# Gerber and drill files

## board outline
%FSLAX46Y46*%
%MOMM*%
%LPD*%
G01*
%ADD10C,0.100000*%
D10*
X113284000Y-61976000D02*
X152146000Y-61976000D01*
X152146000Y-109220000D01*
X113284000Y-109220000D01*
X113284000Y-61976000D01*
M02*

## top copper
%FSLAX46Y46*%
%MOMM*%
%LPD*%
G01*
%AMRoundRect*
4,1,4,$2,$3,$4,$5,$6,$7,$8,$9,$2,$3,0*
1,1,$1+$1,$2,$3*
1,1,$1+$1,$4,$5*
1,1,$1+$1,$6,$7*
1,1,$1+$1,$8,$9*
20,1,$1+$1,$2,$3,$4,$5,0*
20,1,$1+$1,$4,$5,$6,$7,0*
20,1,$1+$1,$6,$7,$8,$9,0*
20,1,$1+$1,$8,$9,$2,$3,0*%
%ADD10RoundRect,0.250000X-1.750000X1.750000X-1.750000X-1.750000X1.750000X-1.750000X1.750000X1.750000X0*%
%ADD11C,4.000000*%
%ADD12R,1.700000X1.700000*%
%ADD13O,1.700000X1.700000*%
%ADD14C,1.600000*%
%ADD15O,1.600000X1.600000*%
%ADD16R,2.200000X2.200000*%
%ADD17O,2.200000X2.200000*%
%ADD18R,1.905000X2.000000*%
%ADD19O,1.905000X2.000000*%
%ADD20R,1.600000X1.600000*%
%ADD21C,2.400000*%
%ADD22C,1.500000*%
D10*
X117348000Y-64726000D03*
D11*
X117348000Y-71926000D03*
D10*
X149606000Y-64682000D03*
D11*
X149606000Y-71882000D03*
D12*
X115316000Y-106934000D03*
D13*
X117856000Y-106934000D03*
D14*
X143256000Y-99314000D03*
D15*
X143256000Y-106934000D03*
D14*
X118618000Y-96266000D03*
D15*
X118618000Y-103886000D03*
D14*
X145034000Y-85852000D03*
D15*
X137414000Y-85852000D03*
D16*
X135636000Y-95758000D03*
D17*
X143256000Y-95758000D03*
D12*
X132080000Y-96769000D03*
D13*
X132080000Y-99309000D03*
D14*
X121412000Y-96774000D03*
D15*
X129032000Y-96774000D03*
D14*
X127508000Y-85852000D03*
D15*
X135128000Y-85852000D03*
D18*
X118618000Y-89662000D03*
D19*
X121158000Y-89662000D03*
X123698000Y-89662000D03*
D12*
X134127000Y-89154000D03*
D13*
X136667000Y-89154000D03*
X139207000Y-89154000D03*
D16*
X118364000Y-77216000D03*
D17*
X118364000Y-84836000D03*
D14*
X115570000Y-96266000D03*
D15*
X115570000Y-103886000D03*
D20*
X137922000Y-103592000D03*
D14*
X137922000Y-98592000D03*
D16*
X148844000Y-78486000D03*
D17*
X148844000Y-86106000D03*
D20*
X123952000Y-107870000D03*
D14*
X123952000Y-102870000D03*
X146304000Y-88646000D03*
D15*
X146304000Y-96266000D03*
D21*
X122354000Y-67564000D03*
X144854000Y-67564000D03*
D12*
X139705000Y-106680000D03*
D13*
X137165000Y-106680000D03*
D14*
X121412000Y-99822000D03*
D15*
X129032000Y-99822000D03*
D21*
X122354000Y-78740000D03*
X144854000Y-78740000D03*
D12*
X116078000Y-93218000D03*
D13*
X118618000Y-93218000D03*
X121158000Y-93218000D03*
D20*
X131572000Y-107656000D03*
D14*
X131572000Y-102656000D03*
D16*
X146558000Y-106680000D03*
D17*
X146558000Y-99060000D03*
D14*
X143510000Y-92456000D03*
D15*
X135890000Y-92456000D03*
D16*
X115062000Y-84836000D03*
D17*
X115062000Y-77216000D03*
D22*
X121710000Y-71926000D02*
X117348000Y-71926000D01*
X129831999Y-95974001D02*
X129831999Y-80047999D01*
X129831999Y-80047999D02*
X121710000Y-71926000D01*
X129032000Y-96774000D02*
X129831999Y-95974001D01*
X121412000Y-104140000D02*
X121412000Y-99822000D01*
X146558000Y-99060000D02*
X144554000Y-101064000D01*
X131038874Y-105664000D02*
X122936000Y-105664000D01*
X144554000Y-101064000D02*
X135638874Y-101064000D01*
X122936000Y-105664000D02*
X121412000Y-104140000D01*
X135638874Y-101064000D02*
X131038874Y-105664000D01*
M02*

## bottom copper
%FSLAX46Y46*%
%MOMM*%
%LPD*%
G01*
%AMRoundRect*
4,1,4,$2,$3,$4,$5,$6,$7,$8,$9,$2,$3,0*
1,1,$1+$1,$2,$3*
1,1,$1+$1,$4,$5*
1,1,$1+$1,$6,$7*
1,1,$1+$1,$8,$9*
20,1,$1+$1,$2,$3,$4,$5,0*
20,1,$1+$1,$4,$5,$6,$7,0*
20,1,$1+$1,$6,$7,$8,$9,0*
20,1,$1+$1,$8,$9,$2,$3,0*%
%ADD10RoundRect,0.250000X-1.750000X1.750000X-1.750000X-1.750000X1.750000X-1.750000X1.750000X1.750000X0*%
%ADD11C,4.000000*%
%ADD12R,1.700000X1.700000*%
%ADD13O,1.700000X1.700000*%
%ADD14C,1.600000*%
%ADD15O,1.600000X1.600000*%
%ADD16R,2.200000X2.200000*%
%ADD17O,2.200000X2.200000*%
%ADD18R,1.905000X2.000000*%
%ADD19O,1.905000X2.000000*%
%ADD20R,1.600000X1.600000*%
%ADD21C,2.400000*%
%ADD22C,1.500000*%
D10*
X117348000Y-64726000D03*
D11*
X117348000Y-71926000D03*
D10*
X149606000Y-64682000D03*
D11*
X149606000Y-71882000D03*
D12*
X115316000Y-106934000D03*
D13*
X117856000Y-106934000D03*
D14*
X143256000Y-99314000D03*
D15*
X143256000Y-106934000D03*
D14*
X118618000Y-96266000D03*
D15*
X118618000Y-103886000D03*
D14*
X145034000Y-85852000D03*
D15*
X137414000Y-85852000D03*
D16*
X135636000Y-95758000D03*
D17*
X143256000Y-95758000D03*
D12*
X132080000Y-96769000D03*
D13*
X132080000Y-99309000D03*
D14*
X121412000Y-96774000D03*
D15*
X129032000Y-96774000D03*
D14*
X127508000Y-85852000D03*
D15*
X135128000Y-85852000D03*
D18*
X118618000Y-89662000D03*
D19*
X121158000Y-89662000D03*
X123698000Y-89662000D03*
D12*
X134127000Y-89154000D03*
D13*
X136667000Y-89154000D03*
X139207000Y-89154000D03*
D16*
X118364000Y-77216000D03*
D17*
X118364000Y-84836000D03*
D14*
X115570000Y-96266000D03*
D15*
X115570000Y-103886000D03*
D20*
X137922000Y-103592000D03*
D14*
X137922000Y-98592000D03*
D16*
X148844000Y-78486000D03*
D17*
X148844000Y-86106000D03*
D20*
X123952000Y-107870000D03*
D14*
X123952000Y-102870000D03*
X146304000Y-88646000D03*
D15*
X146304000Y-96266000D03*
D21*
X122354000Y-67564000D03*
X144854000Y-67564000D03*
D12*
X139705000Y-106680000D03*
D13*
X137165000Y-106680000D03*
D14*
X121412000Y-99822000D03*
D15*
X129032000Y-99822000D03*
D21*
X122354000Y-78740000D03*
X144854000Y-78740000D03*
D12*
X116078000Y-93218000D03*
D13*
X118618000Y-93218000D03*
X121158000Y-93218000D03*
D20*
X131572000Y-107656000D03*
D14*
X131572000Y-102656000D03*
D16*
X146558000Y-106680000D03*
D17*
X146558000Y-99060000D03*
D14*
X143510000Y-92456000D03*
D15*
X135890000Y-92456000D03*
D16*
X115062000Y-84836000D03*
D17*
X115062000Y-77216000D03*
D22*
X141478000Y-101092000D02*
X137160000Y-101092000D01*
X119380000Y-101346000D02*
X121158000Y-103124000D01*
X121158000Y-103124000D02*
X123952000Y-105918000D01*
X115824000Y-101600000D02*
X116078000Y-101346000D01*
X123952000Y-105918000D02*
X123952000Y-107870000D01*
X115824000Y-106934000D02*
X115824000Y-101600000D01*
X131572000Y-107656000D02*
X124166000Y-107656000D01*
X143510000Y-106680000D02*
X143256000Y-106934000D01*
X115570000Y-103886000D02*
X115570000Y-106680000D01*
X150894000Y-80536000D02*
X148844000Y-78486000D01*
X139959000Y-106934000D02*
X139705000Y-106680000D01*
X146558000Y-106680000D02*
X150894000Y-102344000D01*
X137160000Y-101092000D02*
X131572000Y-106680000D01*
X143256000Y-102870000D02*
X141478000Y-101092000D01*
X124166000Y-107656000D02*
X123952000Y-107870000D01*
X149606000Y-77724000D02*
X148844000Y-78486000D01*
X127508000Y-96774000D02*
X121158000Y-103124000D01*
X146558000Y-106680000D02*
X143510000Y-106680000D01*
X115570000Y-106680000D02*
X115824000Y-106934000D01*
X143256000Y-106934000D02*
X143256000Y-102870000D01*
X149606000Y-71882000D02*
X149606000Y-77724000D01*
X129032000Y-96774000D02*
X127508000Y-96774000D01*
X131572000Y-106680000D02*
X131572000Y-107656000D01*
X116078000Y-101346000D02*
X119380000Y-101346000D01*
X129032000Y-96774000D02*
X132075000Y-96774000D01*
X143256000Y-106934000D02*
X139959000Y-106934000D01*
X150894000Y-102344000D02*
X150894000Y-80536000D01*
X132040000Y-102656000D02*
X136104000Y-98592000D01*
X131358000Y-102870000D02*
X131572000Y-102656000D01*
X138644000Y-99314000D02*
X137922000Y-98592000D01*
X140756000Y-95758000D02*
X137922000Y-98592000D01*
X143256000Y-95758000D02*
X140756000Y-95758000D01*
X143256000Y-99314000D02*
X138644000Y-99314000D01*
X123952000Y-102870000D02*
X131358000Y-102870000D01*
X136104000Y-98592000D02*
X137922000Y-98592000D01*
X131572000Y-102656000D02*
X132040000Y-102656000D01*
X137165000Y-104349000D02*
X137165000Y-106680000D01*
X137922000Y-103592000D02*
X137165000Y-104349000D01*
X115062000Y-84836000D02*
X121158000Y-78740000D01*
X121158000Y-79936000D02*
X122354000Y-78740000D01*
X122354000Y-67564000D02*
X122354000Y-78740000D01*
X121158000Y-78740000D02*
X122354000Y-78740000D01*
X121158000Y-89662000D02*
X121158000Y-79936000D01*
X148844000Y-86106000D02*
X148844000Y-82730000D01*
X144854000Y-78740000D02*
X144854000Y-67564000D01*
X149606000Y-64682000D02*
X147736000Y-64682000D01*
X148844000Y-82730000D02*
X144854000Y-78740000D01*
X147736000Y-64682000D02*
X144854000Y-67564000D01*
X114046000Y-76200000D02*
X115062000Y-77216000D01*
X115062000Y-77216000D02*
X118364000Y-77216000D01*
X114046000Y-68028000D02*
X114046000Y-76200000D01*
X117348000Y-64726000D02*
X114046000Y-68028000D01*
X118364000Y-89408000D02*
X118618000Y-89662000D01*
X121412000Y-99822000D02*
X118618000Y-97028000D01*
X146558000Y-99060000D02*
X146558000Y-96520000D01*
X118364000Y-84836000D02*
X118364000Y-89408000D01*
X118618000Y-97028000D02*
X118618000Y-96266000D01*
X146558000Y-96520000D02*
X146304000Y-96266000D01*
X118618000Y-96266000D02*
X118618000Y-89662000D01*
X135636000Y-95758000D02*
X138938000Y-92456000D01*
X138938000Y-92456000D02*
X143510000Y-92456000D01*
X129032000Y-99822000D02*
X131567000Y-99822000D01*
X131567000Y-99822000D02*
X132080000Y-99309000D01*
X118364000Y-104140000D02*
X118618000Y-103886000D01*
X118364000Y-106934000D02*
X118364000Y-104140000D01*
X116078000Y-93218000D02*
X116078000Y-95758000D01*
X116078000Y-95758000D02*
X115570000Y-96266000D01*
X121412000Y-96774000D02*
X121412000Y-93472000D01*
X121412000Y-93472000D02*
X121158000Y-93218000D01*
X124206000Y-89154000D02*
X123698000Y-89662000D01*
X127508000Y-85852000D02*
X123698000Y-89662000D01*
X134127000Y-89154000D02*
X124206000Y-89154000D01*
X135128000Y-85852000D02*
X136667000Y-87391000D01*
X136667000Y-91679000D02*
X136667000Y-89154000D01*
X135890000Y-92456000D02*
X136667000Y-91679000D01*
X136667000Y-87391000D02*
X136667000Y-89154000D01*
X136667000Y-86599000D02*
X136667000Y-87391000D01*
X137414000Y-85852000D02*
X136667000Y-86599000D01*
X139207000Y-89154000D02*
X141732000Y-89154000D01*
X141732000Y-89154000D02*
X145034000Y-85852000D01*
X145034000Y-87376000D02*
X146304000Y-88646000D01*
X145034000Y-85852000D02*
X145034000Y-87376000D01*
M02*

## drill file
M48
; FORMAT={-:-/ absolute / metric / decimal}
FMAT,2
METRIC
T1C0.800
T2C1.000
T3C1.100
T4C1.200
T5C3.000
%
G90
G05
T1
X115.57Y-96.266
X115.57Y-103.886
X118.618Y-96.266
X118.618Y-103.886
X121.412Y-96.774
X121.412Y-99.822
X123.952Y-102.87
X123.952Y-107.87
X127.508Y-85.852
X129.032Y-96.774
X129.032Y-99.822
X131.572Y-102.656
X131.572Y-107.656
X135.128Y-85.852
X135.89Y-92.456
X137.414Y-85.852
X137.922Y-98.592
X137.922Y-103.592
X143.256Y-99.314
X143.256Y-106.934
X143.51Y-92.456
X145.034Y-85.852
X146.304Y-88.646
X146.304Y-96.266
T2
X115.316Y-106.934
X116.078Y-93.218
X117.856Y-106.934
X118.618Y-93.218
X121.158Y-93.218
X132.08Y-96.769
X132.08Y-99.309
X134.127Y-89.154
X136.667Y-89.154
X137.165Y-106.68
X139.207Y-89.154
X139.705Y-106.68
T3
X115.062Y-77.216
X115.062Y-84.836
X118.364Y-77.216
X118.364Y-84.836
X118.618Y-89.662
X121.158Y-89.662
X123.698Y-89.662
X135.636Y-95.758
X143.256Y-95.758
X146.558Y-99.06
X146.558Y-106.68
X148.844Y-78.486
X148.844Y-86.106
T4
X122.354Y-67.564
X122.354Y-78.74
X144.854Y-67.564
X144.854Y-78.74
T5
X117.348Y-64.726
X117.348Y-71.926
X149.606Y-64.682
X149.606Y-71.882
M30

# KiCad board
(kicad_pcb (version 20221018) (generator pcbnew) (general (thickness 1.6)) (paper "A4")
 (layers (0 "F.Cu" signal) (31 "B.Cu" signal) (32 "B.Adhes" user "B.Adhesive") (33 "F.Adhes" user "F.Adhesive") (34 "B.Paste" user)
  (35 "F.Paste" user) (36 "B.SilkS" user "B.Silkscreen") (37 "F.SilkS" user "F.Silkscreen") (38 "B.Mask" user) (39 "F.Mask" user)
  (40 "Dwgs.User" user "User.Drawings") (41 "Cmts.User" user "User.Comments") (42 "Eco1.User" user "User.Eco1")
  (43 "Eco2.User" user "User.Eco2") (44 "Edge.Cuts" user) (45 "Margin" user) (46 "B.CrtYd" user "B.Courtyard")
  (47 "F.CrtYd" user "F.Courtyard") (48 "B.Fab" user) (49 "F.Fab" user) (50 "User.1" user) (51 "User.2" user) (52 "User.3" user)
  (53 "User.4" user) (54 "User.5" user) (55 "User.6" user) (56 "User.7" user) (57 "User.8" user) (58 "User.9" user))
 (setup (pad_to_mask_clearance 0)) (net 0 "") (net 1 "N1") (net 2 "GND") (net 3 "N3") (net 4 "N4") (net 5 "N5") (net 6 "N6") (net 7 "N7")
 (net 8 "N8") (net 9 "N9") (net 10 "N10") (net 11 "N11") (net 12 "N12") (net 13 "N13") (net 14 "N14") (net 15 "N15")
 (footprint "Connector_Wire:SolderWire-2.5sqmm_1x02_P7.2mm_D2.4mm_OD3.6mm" (layer "F.Cu") (at 117.348 64.726 -90)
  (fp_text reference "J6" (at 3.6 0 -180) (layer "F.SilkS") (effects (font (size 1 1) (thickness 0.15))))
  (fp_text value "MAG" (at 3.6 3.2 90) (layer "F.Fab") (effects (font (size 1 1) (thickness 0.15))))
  (pad "1" thru_hole roundrect (at 0 0 270) (size 4 4) (drill 3) (layers "*.Cu" "*.Mask") (roundrect_rratio 0.0625) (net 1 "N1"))
  (pad "2" thru_hole circle (at 7.2 0 270) (size 4 4) (drill 3) (layers "*.Cu" "*.Mask") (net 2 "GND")))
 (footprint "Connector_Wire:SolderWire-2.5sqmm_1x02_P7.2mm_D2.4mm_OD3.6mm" (layer "F.Cu") (at 149.606 64.682 -90)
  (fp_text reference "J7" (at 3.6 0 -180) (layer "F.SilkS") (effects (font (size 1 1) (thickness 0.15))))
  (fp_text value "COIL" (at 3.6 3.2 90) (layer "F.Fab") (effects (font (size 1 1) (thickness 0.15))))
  (pad "1" thru_hole roundrect (at 0 0 270) (size 4 4) (drill 3) (layers "*.Cu" "*.Mask") (roundrect_rratio 0.0625) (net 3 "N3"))
  (pad "2" thru_hole circle (at 7.2 0 270) (size 4 4) (drill 3) (layers "*.Cu" "*.Mask") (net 2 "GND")))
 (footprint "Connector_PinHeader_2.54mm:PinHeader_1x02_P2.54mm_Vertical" (layer "F.Cu") (at 115.316 106.934 90)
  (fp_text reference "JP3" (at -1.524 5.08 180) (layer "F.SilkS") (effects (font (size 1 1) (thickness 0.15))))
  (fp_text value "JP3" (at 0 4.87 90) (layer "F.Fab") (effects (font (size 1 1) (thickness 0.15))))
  (pad "1" thru_hole rect (at 0 0 90) (size 1.7 1.7) (drill 1) (layers "*.Cu" "*.Mask") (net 2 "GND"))
  (pad "2" thru_hole oval (at 0 2.54 90) (size 1.7 1.7) (drill 1) (layers "*.Cu" "*.Mask") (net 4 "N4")))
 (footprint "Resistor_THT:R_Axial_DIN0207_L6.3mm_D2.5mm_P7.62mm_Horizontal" (layer "F.Cu") (at 143.256 99.314 -90)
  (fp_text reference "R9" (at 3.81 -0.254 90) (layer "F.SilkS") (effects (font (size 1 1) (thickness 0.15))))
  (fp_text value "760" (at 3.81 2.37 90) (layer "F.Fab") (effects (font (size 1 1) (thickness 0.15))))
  (pad "1" thru_hole circle (at 0 0 270) (size 1.6 1.6) (drill 0.8) (layers "*.Cu" "*.Mask") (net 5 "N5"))
  (pad "2" thru_hole oval (at 7.62 0 270) (size 1.6 1.6) (drill 0.8) (layers "*.Cu" "*.Mask") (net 2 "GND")))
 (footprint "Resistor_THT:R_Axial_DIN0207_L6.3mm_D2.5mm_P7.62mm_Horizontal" (layer "F.Cu") (at 118.618 96.266 -90)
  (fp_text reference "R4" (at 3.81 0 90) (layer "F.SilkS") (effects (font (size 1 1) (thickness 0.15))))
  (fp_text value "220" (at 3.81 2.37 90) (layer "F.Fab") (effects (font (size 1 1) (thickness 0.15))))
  (pad "1" thru_hole circle (at 0 0 270) (size 1.6 1.6) (drill 0.8) (layers "*.Cu" "*.Mask") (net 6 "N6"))
  (pad "2" thru_hole oval (at 7.62 0 270) (size 1.6 1.6) (drill 0.8) (layers "*.Cu" "*.Mask") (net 4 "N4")))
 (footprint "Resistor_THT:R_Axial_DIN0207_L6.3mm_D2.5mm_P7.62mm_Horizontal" (layer "F.Cu") (at 145.034 85.852 180)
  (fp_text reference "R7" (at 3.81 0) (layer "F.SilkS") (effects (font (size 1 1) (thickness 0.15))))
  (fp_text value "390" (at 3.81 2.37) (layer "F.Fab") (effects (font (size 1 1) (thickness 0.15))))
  (pad "1" thru_hole circle (at 0 0 180) (size 1.6 1.6) (drill 0.8) (layers "*.Cu" "*.Mask") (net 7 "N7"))
  (pad "2" thru_hole oval (at 7.62 0 180) (size 1.6 1.6) (drill 0.8) (layers "*.Cu" "*.Mask") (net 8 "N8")))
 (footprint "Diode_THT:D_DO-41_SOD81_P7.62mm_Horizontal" (layer "F.Cu") (at 135.636 95.758)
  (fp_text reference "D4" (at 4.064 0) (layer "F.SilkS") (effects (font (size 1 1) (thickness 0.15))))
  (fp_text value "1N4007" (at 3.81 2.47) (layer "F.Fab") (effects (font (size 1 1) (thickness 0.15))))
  (pad "1" thru_hole rect (at 0 0) (size 2.2 2.2) (drill 1.1) (layers "*.Cu" "*.Mask") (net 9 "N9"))
  (pad "2" thru_hole oval (at 7.62 0) (size 2.2 2.2) (drill 1.1) (layers "*.Cu" "*.Mask") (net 5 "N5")))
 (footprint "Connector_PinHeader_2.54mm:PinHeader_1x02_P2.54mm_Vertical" (layer "F.Cu") (at 132.08 96.769)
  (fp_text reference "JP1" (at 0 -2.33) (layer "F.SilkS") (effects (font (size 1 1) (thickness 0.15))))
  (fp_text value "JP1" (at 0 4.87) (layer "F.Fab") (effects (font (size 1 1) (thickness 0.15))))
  (pad "1" thru_hole rect (at 0 0) (size 1.7 1.7) (drill 1) (layers "*.Cu" "*.Mask") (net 2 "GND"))
  (pad "2" thru_hole oval (at 0 2.54) (size 1.7 1.7) (drill 1) (layers "*.Cu" "*.Mask") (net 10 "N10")))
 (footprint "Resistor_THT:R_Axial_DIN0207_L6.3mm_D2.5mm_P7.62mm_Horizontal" (layer "F.Cu") (at 121.412 96.774)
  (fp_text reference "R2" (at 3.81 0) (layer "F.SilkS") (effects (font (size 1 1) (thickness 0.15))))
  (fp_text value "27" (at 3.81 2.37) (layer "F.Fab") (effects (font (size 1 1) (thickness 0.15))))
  (pad "1" thru_hole circle (at 0 0) (size 1.6 1.6) (drill 0.8) (layers "*.Cu" "*.Mask") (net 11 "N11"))
  (pad "2" thru_hole oval (at 7.62 0) (size 1.6 1.6) (drill 0.8) (layers "*.Cu" "*.Mask") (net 2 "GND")))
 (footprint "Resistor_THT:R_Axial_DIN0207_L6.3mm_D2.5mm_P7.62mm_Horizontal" (layer "F.Cu") (at 127.508 85.852)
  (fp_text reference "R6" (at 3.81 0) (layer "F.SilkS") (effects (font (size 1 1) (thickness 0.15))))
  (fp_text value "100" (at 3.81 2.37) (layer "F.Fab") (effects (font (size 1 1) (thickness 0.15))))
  (pad "1" thru_hole circle (at 0 0) (size 1.6 1.6) (drill 0.8) (layers "*.Cu" "*.Mask") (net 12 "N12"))
  (pad "2" thru_hole oval (at 7.62 0) (size 1.6 1.6) (drill 0.8) (layers "*.Cu" "*.Mask") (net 8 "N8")))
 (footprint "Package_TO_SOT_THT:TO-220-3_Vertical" (layer "F.Cu") (at 118.618 89.662)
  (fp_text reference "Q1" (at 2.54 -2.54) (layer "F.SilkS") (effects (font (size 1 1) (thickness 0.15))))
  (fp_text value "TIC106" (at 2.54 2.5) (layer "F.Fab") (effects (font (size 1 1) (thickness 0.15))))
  (pad "1" thru_hole rect (at 0 0) (size 1.905 2) (drill 1.1) (layers "*.Cu" "*.Mask") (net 6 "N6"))
  (pad "2" thru_hole oval (at 2.54 0) (size 1.905 2) (drill 1.1) (layers "*.Cu" "*.Mask") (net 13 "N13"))
  (pad "3" thru_hole oval (at 5.08 0) (size 1.905 2) (drill 1.1) (layers "*.Cu" "*.Mask") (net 12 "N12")))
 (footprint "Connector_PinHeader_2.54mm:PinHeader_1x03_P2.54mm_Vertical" (layer "F.Cu") (at 134.127 89.154 90)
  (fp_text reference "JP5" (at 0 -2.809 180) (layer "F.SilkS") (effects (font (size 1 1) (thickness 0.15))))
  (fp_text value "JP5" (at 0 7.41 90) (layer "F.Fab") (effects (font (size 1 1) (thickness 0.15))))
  (pad "1" thru_hole rect (at 0 0 90) (size 1.7 1.7) (drill 1) (layers "*.Cu" "*.Mask") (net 12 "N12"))
  (pad "2" thru_hole oval (at 0 2.54 90) (size 1.7 1.7) (drill 1) (layers "*.Cu" "*.Mask") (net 8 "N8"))
  (pad "3" thru_hole oval (at 0 5.08 90) (size 1.7 1.7) (drill 1) (layers "*.Cu" "*.Mask") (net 7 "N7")))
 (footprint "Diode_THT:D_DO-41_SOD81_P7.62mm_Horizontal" (layer "F.Cu") (at 118.364 77.216 -90)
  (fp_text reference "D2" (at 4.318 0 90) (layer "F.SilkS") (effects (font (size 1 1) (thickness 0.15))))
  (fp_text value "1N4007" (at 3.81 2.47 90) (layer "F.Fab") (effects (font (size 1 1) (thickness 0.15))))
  (pad "1" thru_hole rect (at 0 0 270) (size 2.2 2.2) (drill 1.1) (layers "*.Cu" "*.Mask") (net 1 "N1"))
  (pad "2" thru_hole oval (at 7.62 0 270) (size 2.2 2.2) (drill 1.1) (layers "*.Cu" "*.Mask") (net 6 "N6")))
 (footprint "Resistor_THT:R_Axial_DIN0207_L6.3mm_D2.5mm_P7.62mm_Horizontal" (layer "F.Cu") (at 115.57 96.266 -90)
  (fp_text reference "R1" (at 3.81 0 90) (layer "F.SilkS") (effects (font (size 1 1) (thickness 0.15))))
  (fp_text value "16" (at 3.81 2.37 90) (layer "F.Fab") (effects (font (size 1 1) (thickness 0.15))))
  (pad "1" thru_hole circle (at 0 0 270) (size 1.6 1.6) (drill 0.8) (layers "*.Cu" "*.Mask") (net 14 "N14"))
  (pad "2" thru_hole oval (at 7.62 0 270) (size 1.6 1.6) (drill 0.8) (layers "*.Cu" "*.Mask") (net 2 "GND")))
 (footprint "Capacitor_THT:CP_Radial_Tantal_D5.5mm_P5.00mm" (layer "F.Cu") (at 137.922 103.592 90)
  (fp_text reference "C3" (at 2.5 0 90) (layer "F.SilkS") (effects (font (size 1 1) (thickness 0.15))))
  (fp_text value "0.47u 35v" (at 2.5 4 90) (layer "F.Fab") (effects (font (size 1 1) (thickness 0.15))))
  (pad "1" thru_hole rect (at 0 0 90) (size 1.6 1.6) (drill 0.8) (layers "*.Cu" "*.Mask") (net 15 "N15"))
  (pad "2" thru_hole circle (at 5 0 90) (size 1.6 1.6) (drill 0.8) (layers "*.Cu" "*.Mask") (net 5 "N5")))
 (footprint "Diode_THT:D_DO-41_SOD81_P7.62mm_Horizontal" (layer "F.Cu") (at 148.844 78.486 -90)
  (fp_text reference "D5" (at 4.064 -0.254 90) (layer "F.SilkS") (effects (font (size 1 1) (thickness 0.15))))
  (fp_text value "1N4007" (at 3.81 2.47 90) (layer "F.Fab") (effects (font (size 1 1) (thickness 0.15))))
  (pad "1" thru_hole rect (at 0 0 270) (size 2.2 2.2) (drill 1.1) (layers "*.Cu" "*.Mask") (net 2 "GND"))
  (pad "2" thru_hole oval (at 7.62 0 270) (size 2.2 2.2) (drill 1.1) (layers "*.Cu" "*.Mask") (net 3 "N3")))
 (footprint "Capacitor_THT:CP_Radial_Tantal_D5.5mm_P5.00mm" (layer "F.Cu") (at 123.952 107.87 90)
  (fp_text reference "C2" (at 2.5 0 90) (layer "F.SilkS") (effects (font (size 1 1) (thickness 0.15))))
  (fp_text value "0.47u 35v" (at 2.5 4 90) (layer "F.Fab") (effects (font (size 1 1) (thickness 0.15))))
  (pad "1" thru_hole rect (at 0 0 90) (size 1.6 1.6) (drill 0.8) (layers "*.Cu" "*.Mask") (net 2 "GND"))
  (pad "2" thru_hole circle (at 5 0 90) (size 1.6 1.6) (drill 0.8) (layers "*.Cu" "*.Mask") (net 5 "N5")))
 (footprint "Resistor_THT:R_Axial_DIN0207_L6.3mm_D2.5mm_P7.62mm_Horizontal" (layer "F.Cu") (at 146.304 88.646 -90)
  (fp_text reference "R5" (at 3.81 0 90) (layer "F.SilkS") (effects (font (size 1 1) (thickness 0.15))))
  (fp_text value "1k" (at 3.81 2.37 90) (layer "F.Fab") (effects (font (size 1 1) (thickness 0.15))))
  (pad "1" thru_hole circle (at 0 0 270) (size 1.6 1.6) (drill 0.8) (layers "*.Cu" "*.Mask") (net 7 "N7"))
  (pad "2" thru_hole oval (at 7.62 0 270) (size 1.6 1.6) (drill 0.8) (layers "*.Cu" "*.Mask") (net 6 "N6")))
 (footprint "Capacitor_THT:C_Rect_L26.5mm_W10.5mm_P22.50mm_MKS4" (layer "F.Cu") (at 122.354 67.564)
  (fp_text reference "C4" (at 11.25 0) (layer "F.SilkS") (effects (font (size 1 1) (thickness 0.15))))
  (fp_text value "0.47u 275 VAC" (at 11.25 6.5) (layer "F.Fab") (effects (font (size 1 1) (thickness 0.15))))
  (pad "1" thru_hole circle (at 0 0) (size 2.4 2.4) (drill 1.2) (layers "*.Cu" "*.Mask") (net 13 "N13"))
  (pad "2" thru_hole circle (at 22.5 0) (size 2.4 2.4) (drill 1.2) (layers "*.Cu" "*.Mask") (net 3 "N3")))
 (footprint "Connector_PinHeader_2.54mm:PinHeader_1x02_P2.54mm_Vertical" (layer "F.Cu") (at 139.705 106.68 -90)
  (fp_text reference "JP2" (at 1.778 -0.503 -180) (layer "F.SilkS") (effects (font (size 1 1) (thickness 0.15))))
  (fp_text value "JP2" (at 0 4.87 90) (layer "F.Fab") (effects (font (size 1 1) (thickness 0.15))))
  (pad "1" thru_hole rect (at 0 0 270) (size 1.7 1.7) (drill 1) (layers "*.Cu" "*.Mask") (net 2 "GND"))
  (pad "2" thru_hole oval (at 0 2.54 270) (size 1.7 1.7) (drill 1) (layers "*.Cu" "*.Mask") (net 15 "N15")))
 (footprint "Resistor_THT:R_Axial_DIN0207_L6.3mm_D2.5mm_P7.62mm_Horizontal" (layer "F.Cu") (at 121.412 99.822)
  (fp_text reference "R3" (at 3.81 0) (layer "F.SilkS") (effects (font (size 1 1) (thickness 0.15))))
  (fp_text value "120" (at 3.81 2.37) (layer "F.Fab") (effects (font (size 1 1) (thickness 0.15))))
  (pad "1" thru_hole circle (at 0 0) (size 1.6 1.6) (drill 0.8) (layers "*.Cu" "*.Mask") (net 6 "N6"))
  (pad "2" thru_hole oval (at 7.62 0) (size 1.6 1.6) (drill 0.8) (layers "*.Cu" "*.Mask") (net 10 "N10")))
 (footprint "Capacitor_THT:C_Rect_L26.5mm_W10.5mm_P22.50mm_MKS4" (layer "F.Cu") (at 122.354 78.74)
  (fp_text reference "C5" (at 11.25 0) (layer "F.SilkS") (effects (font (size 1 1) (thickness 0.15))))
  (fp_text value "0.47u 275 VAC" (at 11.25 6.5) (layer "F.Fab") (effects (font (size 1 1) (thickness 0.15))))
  (pad "1" thru_hole circle (at 0 0) (size 2.4 2.4) (drill 1.2) (layers "*.Cu" "*.Mask") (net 13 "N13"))
  (pad "2" thru_hole circle (at 22.5 0) (size 2.4 2.4) (drill 1.2) (layers "*.Cu" "*.Mask") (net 3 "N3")))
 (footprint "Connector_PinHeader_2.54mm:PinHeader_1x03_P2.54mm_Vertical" (layer "F.Cu") (at 116.078 93.218 90)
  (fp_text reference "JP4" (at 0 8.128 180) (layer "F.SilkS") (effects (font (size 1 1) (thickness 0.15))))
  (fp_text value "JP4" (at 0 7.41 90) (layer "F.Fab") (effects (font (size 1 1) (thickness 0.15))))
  (pad "1" thru_hole rect (at 0 0 90) (size 1.7 1.7) (drill 1) (layers "*.Cu" "*.Mask") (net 14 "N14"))
  (pad "2" thru_hole oval (at 0 2.54 90) (size 1.7 1.7) (drill 1) (layers "*.Cu" "*.Mask") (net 6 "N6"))
  (pad "3" thru_hole oval (at 0 5.08 90) (size 1.7 1.7) (drill 1) (layers "*.Cu" "*.Mask") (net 11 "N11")))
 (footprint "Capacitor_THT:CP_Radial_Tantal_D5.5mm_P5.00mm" (layer "F.Cu") (at 131.572 107.656 90)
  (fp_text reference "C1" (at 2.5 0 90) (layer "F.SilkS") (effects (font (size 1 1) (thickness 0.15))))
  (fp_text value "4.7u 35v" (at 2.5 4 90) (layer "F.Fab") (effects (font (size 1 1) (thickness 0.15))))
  (pad "1" thru_hole rect (at 0 0 90) (size 1.6 1.6) (drill 0.8) (layers "*.Cu" "*.Mask") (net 2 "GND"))
  (pad "2" thru_hole circle (at 5 0 90) (size 1.6 1.6) (drill 0.8) (layers "*.Cu" "*.Mask") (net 5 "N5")))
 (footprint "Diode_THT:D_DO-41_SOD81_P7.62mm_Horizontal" (layer "F.Cu") (at 146.558 106.68 90)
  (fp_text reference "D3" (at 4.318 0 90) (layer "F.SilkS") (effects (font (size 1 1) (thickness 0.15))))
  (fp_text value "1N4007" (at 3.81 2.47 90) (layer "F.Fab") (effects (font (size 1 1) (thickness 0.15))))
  (pad "1" thru_hole rect (at 0 0 90) (size 2.2 2.2) (drill 1.1) (layers "*.Cu" "*.Mask") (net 2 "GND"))
  (pad "2" thru_hole oval (at 7.62 0 90) (size 2.2 2.2) (drill 1.1) (layers "*.Cu" "*.Mask") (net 6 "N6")))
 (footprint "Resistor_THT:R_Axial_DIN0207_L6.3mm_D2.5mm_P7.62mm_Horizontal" (layer "F.Cu") (at 143.51 92.456 180)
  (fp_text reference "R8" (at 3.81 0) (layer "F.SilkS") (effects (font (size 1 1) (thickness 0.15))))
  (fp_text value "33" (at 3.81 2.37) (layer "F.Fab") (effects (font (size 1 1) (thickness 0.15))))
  (pad "1" thru_hole circle (at 0 0 180) (size 1.6 1.6) (drill 0.8) (layers "*.Cu" "*.Mask") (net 9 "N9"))
  (pad "2" thru_hole oval (at 7.62 0 180) (size 1.6 1.6) (drill 0.8) (layers "*.Cu" "*.Mask") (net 8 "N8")))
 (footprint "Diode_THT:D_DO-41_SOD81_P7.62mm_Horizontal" (layer "F.Cu") (at 115.062 84.836 90)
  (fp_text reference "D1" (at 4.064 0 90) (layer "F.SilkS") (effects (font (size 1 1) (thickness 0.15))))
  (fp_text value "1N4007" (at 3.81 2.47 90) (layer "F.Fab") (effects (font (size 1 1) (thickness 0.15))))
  (pad "1" thru_hole rect (at 0 0 90) (size 2.2 2.2) (drill 1.1) (layers "*.Cu" "*.Mask") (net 13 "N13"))
  (pad "2" thru_hole oval (at 7.62 0 90) (size 2.2 2.2) (drill 1.1) (layers "*.Cu" "*.Mask") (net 1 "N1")))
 (gr_rect (start 113.284 61.976) (end 152.146 109.22) (stroke (width 0.1) (type default)) (fill none) (layer "Edge.Cuts"))
 (segment (start 121.71 71.926) (end 117.348 71.926) (width 1.5) (layer "F.Cu") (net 2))
 (segment (start 129.831999 95.974001) (end 129.831999 80.047999) (width 1.5) (layer "F.Cu") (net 2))
 (segment (start 129.831999 80.047999) (end 121.71 71.926) (width 1.5) (layer "F.Cu") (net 2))
 (segment (start 129.032 96.774) (end 129.831999 95.974001) (width 1.5) (layer "F.Cu") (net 2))
 (segment (start 141.478 101.092) (end 137.16 101.092) (width 1.5) (layer "B.Cu") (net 2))
 (segment (start 119.38 101.346) (end 121.158 103.124) (width 1.5) (layer "B.Cu") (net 2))
 (segment (start 121.158 103.124) (end 123.952 105.918) (width 1.5) (layer "B.Cu") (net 2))
 (segment (start 115.824 101.6) (end 116.078 101.346) (width 1.5) (layer "B.Cu") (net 2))
 (segment (start 123.952 105.918) (end 123.952 107.87) (width 1.5) (layer "B.Cu") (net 2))
 (segment (start 115.824 106.934) (end 115.824 101.6) (width 1.5) (layer "B.Cu") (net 2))
 (segment (start 131.572 107.656) (end 124.166 107.656) (width 1.5) (layer "B.Cu") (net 2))
 (segment (start 143.51 106.68) (end 143.256 106.934) (width 1.5) (layer "B.Cu") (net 2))
 (segment (start 115.57 103.886) (end 115.57 106.68) (width 1.5) (layer "B.Cu") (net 2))
 (segment (start 150.894 80.536) (end 148.844 78.486) (width 1.5) (layer "B.Cu") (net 2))
 (segment (start 139.959 106.934) (end 139.705 106.68) (width 1.5) (layer "B.Cu") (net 2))
 (segment (start 146.558 106.68) (end 150.894 102.344) (width 1.5) (layer "B.Cu") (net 2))
 (segment (start 137.16 101.092) (end 131.572 106.68) (width 1.5) (layer "B.Cu") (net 2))
 (segment (start 143.256 102.87) (end 141.478 101.092) (width 1.5) (layer "B.Cu") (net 2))
 (segment (start 124.166 107.656) (end 123.952 107.87) (width 1.5) (layer "B.Cu") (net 2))
 (segment (start 149.606 77.724) (end 148.844 78.486) (width 1.5) (layer "B.Cu") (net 2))
 (segment (start 127.508 96.774) (end 121.158 103.124) (width 1.5) (layer "B.Cu") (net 2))
 (segment (start 146.558 106.68) (end 143.51 106.68) (width 1.5) (layer "B.Cu") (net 2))
 (segment (start 115.57 106.68) (end 115.824 106.934) (width 1.5) (layer "B.Cu") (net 2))
 (segment (start 143.256 106.934) (end 143.256 102.87) (width 1.5) (layer "B.Cu") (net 2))
 (segment (start 149.606 71.882) (end 149.606 77.724) (width 1.5) (layer "B.Cu") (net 2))
 (segment (start 129.032 96.774) (end 127.508 96.774) (width 1.5) (layer "B.Cu") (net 2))
 (segment (start 131.572 106.68) (end 131.572 107.656) (width 1.5) (layer "B.Cu") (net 2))
 (segment (start 116.078 101.346) (end 119.38 101.346) (width 1.5) (layer "B.Cu") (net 2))
 (segment (start 129.032 96.774) (end 132.075 96.774) (width 1.5) (layer "B.Cu") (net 2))
 (segment (start 143.256 106.934) (end 139.959 106.934) (width 1.5) (layer "B.Cu") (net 2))
 (segment (start 150.894 102.344) (end 150.894 80.536) (width 1.5) (layer "B.Cu") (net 2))
 (segment (start 132.04 102.656) (end 136.104 98.592) (width 1.5) (layer "B.Cu") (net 5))
 (segment (start 131.358 102.87) (end 131.572 102.656) (width 1.5) (layer "B.Cu") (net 5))
 (segment (start 138.644 99.314) (end 137.922 98.592) (width 1.5) (layer "B.Cu") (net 5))
 (segment (start 140.756 95.758) (end 137.922 98.592) (width 1.5) (layer "B.Cu") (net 5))
 (segment (start 143.256 95.758) (end 140.756 95.758) (width 1.5) (layer "B.Cu") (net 5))
 (segment (start 143.256 99.314) (end 138.644 99.314) (width 1.5) (layer "B.Cu") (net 5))
 (segment (start 123.952 102.87) (end 131.358 102.87) (width 1.5) (layer "B.Cu") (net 5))
 (segment (start 136.104 98.592) (end 137.922 98.592) (width 1.5) (layer "B.Cu") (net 5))
 (segment (start 131.572 102.656) (end 132.04 102.656) (width 1.5) (layer "B.Cu") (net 5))
 (segment (start 137.165 104.349) (end 137.165 106.68) (width 1.5) (layer "B.Cu") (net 15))
 (segment (start 137.922 103.592) (end 137.165 104.349) (width 1.5) (layer "B.Cu") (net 15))
 (segment (start 115.062 84.836) (end 121.158 78.74) (width 1.5) (layer "B.Cu") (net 13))
 (segment (start 121.158 79.936) (end 122.354 78.74) (width 1.5) (layer "B.Cu") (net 13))
 (segment (start 122.354 67.564) (end 122.354 78.74) (width 1.5) (layer "B.Cu") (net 13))
 (segment (start 121.158 78.74) (end 122.354 78.74) (width 1.5) (layer "B.Cu") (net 13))
 (segment (start 121.158 89.662) (end 121.158 79.936) (width 1.5) (layer "B.Cu") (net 13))
 (segment (start 148.844 86.106) (end 148.844 82.73) (width 1.5) (layer "B.Cu") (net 3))
 (segment (start 144.854 78.74) (end 144.854 67.564) (width 1.5) (layer "B.Cu") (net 3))
 (segment (start 149.606 64.682) (end 147.736 64.682) (width 1.5) (layer "B.Cu") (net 3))
 (segment (start 148.844 82.73) (end 144.854 78.74) (width 1.5) (layer "B.Cu") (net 3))
 (segment (start 147.736 64.682) (end 144.854 67.564) (width 1.5) (layer "B.Cu") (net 3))
 (segment (start 114.046 76.2) (end 115.062 77.216) (width 1.5) (layer "B.Cu") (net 1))
 (segment (start 115.062 77.216) (end 118.364 77.216) (width 1.5) (layer "B.Cu") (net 1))
 (segment (start 114.046 68.028) (end 114.046 76.2) (width 1.5) (layer "B.Cu") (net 1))
 (segment (start 117.348 64.726) (end 114.046 68.028) (width 1.5) (layer "B.Cu") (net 1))
 (segment (start 121.412 104.14) (end 121.412 99.822) (width 1.5) (layer "F.Cu") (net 6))
 (segment (start 146.558 99.06) (end 144.554 101.064) (width 1.5) (layer "F.Cu") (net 6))
 (segment (start 131.038874 105.664) (end 122.936 105.664) (width 1.5) (layer "F.Cu") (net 6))
 (segment (start 144.554 101.064) (end 135.638874 101.064) (width 1.5) (layer "F.Cu") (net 6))
 (segment (start 122.936 105.664) (end 121.412 104.14) (width 1.5) (layer "F.Cu") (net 6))
 (segment (start 135.638874 101.064) (end 131.038874 105.664) (width 1.5) (layer "F.Cu") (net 6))
 (segment (start 118.364 89.408) (end 118.618 89.662) (width 1.5) (layer "B.Cu") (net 6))
 (segment (start 121.412 99.822) (end 118.618 97.028) (width 1.5) (layer "B.Cu") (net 6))
 (segment (start 146.558 99.06) (end 146.558 96.52) (width 1.5) (layer "B.Cu") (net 6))
 (segment (start 118.364 84.836) (end 118.364 89.408) (width 1.5) (layer "B.Cu") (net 6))
 (segment (start 118.618 97.028) (end 118.618 96.266) (width 1.5) (layer "B.Cu") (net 6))
 (segment (start 146.558 96.52) (end 146.304 96.266) (width 1.5) (layer "B.Cu") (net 6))
 (segment (start 118.618 96.266) (end 118.618 89.662) (width 1.5) (layer "B.Cu") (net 6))
 (segment (start 135.636 95.758) (end 138.938 92.456) (width 1.5) (layer "B.Cu") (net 9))
 (segment (start 138.938 92.456) (end 143.51 92.456) (width 1.5) (layer "B.Cu") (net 9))
 (segment (start 129.032 99.822) (end 131.567 99.822) (width 1.5) (layer "B.Cu") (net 10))
 (segment (start 131.567 99.822) (end 132.08 99.309) (width 1.5) (layer "B.Cu") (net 10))
 (segment (start 118.364 104.14) (end 118.618 103.886) (width 1.5) (layer "B.Cu") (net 4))
 (segment (start 118.364 106.934) (end 118.364 104.14) (width 1.5) (layer "B.Cu") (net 4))
 (segment (start 116.078 93.218) (end 116.078 95.758) (width 1.5) (layer "B.Cu") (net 14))
 (segment (start 116.078 95.758) (end 115.57 96.266) (width 1.5) (layer "B.Cu") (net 14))
 (segment (start 121.412 96.774) (end 121.412 93.472) (width 1.5) (layer "B.Cu") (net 11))
 (segment (start 121.412 93.472) (end 121.158 93.218) (width 1.5) (layer "B.Cu") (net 11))
 (segment (start 124.206 89.154) (end 123.698 89.662) (width 1.5) (layer "B.Cu") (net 12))
 (segment (start 127.508 85.852) (end 123.698 89.662) (width 1.5) (layer "B.Cu") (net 12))
 (segment (start 134.127 89.154) (end 124.206 89.154) (width 1.5) (layer "B.Cu") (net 12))
 (segment (start 135.128 85.852) (end 136.667 87.391) (width 1.5) (layer "B.Cu") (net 8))
 (segment (start 136.667 91.679) (end 136.667 89.154) (width 1.5) (layer "B.Cu") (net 8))
 (segment (start 135.89 92.456) (end 136.667 91.679) (width 1.5) (layer "B.Cu") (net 8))
 (segment (start 136.667 87.391) (end 136.667 89.154) (width 1.5) (layer "B.Cu") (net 8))
 (segment (start 136.667 86.599) (end 136.667 87.391) (width 1.5) (layer "B.Cu") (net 8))
 (segment (start 137.414 85.852) (end 136.667 86.599) (width 1.5) (layer "B.Cu") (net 8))
 (segment (start 139.207 89.154) (end 141.732 89.154) (width 1.5) (layer "B.Cu") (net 7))
 (segment (start 141.732 89.154) (end 145.034 85.852) (width 1.5) (layer "B.Cu") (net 7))
 (segment (start 145.034 87.376) (end 146.304 88.646) (width 1.5) (layer "B.Cu") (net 7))
 (segment (start 145.034 85.852) (end 145.034 87.376) (width 1.5) (layer "B.Cu") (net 7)))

